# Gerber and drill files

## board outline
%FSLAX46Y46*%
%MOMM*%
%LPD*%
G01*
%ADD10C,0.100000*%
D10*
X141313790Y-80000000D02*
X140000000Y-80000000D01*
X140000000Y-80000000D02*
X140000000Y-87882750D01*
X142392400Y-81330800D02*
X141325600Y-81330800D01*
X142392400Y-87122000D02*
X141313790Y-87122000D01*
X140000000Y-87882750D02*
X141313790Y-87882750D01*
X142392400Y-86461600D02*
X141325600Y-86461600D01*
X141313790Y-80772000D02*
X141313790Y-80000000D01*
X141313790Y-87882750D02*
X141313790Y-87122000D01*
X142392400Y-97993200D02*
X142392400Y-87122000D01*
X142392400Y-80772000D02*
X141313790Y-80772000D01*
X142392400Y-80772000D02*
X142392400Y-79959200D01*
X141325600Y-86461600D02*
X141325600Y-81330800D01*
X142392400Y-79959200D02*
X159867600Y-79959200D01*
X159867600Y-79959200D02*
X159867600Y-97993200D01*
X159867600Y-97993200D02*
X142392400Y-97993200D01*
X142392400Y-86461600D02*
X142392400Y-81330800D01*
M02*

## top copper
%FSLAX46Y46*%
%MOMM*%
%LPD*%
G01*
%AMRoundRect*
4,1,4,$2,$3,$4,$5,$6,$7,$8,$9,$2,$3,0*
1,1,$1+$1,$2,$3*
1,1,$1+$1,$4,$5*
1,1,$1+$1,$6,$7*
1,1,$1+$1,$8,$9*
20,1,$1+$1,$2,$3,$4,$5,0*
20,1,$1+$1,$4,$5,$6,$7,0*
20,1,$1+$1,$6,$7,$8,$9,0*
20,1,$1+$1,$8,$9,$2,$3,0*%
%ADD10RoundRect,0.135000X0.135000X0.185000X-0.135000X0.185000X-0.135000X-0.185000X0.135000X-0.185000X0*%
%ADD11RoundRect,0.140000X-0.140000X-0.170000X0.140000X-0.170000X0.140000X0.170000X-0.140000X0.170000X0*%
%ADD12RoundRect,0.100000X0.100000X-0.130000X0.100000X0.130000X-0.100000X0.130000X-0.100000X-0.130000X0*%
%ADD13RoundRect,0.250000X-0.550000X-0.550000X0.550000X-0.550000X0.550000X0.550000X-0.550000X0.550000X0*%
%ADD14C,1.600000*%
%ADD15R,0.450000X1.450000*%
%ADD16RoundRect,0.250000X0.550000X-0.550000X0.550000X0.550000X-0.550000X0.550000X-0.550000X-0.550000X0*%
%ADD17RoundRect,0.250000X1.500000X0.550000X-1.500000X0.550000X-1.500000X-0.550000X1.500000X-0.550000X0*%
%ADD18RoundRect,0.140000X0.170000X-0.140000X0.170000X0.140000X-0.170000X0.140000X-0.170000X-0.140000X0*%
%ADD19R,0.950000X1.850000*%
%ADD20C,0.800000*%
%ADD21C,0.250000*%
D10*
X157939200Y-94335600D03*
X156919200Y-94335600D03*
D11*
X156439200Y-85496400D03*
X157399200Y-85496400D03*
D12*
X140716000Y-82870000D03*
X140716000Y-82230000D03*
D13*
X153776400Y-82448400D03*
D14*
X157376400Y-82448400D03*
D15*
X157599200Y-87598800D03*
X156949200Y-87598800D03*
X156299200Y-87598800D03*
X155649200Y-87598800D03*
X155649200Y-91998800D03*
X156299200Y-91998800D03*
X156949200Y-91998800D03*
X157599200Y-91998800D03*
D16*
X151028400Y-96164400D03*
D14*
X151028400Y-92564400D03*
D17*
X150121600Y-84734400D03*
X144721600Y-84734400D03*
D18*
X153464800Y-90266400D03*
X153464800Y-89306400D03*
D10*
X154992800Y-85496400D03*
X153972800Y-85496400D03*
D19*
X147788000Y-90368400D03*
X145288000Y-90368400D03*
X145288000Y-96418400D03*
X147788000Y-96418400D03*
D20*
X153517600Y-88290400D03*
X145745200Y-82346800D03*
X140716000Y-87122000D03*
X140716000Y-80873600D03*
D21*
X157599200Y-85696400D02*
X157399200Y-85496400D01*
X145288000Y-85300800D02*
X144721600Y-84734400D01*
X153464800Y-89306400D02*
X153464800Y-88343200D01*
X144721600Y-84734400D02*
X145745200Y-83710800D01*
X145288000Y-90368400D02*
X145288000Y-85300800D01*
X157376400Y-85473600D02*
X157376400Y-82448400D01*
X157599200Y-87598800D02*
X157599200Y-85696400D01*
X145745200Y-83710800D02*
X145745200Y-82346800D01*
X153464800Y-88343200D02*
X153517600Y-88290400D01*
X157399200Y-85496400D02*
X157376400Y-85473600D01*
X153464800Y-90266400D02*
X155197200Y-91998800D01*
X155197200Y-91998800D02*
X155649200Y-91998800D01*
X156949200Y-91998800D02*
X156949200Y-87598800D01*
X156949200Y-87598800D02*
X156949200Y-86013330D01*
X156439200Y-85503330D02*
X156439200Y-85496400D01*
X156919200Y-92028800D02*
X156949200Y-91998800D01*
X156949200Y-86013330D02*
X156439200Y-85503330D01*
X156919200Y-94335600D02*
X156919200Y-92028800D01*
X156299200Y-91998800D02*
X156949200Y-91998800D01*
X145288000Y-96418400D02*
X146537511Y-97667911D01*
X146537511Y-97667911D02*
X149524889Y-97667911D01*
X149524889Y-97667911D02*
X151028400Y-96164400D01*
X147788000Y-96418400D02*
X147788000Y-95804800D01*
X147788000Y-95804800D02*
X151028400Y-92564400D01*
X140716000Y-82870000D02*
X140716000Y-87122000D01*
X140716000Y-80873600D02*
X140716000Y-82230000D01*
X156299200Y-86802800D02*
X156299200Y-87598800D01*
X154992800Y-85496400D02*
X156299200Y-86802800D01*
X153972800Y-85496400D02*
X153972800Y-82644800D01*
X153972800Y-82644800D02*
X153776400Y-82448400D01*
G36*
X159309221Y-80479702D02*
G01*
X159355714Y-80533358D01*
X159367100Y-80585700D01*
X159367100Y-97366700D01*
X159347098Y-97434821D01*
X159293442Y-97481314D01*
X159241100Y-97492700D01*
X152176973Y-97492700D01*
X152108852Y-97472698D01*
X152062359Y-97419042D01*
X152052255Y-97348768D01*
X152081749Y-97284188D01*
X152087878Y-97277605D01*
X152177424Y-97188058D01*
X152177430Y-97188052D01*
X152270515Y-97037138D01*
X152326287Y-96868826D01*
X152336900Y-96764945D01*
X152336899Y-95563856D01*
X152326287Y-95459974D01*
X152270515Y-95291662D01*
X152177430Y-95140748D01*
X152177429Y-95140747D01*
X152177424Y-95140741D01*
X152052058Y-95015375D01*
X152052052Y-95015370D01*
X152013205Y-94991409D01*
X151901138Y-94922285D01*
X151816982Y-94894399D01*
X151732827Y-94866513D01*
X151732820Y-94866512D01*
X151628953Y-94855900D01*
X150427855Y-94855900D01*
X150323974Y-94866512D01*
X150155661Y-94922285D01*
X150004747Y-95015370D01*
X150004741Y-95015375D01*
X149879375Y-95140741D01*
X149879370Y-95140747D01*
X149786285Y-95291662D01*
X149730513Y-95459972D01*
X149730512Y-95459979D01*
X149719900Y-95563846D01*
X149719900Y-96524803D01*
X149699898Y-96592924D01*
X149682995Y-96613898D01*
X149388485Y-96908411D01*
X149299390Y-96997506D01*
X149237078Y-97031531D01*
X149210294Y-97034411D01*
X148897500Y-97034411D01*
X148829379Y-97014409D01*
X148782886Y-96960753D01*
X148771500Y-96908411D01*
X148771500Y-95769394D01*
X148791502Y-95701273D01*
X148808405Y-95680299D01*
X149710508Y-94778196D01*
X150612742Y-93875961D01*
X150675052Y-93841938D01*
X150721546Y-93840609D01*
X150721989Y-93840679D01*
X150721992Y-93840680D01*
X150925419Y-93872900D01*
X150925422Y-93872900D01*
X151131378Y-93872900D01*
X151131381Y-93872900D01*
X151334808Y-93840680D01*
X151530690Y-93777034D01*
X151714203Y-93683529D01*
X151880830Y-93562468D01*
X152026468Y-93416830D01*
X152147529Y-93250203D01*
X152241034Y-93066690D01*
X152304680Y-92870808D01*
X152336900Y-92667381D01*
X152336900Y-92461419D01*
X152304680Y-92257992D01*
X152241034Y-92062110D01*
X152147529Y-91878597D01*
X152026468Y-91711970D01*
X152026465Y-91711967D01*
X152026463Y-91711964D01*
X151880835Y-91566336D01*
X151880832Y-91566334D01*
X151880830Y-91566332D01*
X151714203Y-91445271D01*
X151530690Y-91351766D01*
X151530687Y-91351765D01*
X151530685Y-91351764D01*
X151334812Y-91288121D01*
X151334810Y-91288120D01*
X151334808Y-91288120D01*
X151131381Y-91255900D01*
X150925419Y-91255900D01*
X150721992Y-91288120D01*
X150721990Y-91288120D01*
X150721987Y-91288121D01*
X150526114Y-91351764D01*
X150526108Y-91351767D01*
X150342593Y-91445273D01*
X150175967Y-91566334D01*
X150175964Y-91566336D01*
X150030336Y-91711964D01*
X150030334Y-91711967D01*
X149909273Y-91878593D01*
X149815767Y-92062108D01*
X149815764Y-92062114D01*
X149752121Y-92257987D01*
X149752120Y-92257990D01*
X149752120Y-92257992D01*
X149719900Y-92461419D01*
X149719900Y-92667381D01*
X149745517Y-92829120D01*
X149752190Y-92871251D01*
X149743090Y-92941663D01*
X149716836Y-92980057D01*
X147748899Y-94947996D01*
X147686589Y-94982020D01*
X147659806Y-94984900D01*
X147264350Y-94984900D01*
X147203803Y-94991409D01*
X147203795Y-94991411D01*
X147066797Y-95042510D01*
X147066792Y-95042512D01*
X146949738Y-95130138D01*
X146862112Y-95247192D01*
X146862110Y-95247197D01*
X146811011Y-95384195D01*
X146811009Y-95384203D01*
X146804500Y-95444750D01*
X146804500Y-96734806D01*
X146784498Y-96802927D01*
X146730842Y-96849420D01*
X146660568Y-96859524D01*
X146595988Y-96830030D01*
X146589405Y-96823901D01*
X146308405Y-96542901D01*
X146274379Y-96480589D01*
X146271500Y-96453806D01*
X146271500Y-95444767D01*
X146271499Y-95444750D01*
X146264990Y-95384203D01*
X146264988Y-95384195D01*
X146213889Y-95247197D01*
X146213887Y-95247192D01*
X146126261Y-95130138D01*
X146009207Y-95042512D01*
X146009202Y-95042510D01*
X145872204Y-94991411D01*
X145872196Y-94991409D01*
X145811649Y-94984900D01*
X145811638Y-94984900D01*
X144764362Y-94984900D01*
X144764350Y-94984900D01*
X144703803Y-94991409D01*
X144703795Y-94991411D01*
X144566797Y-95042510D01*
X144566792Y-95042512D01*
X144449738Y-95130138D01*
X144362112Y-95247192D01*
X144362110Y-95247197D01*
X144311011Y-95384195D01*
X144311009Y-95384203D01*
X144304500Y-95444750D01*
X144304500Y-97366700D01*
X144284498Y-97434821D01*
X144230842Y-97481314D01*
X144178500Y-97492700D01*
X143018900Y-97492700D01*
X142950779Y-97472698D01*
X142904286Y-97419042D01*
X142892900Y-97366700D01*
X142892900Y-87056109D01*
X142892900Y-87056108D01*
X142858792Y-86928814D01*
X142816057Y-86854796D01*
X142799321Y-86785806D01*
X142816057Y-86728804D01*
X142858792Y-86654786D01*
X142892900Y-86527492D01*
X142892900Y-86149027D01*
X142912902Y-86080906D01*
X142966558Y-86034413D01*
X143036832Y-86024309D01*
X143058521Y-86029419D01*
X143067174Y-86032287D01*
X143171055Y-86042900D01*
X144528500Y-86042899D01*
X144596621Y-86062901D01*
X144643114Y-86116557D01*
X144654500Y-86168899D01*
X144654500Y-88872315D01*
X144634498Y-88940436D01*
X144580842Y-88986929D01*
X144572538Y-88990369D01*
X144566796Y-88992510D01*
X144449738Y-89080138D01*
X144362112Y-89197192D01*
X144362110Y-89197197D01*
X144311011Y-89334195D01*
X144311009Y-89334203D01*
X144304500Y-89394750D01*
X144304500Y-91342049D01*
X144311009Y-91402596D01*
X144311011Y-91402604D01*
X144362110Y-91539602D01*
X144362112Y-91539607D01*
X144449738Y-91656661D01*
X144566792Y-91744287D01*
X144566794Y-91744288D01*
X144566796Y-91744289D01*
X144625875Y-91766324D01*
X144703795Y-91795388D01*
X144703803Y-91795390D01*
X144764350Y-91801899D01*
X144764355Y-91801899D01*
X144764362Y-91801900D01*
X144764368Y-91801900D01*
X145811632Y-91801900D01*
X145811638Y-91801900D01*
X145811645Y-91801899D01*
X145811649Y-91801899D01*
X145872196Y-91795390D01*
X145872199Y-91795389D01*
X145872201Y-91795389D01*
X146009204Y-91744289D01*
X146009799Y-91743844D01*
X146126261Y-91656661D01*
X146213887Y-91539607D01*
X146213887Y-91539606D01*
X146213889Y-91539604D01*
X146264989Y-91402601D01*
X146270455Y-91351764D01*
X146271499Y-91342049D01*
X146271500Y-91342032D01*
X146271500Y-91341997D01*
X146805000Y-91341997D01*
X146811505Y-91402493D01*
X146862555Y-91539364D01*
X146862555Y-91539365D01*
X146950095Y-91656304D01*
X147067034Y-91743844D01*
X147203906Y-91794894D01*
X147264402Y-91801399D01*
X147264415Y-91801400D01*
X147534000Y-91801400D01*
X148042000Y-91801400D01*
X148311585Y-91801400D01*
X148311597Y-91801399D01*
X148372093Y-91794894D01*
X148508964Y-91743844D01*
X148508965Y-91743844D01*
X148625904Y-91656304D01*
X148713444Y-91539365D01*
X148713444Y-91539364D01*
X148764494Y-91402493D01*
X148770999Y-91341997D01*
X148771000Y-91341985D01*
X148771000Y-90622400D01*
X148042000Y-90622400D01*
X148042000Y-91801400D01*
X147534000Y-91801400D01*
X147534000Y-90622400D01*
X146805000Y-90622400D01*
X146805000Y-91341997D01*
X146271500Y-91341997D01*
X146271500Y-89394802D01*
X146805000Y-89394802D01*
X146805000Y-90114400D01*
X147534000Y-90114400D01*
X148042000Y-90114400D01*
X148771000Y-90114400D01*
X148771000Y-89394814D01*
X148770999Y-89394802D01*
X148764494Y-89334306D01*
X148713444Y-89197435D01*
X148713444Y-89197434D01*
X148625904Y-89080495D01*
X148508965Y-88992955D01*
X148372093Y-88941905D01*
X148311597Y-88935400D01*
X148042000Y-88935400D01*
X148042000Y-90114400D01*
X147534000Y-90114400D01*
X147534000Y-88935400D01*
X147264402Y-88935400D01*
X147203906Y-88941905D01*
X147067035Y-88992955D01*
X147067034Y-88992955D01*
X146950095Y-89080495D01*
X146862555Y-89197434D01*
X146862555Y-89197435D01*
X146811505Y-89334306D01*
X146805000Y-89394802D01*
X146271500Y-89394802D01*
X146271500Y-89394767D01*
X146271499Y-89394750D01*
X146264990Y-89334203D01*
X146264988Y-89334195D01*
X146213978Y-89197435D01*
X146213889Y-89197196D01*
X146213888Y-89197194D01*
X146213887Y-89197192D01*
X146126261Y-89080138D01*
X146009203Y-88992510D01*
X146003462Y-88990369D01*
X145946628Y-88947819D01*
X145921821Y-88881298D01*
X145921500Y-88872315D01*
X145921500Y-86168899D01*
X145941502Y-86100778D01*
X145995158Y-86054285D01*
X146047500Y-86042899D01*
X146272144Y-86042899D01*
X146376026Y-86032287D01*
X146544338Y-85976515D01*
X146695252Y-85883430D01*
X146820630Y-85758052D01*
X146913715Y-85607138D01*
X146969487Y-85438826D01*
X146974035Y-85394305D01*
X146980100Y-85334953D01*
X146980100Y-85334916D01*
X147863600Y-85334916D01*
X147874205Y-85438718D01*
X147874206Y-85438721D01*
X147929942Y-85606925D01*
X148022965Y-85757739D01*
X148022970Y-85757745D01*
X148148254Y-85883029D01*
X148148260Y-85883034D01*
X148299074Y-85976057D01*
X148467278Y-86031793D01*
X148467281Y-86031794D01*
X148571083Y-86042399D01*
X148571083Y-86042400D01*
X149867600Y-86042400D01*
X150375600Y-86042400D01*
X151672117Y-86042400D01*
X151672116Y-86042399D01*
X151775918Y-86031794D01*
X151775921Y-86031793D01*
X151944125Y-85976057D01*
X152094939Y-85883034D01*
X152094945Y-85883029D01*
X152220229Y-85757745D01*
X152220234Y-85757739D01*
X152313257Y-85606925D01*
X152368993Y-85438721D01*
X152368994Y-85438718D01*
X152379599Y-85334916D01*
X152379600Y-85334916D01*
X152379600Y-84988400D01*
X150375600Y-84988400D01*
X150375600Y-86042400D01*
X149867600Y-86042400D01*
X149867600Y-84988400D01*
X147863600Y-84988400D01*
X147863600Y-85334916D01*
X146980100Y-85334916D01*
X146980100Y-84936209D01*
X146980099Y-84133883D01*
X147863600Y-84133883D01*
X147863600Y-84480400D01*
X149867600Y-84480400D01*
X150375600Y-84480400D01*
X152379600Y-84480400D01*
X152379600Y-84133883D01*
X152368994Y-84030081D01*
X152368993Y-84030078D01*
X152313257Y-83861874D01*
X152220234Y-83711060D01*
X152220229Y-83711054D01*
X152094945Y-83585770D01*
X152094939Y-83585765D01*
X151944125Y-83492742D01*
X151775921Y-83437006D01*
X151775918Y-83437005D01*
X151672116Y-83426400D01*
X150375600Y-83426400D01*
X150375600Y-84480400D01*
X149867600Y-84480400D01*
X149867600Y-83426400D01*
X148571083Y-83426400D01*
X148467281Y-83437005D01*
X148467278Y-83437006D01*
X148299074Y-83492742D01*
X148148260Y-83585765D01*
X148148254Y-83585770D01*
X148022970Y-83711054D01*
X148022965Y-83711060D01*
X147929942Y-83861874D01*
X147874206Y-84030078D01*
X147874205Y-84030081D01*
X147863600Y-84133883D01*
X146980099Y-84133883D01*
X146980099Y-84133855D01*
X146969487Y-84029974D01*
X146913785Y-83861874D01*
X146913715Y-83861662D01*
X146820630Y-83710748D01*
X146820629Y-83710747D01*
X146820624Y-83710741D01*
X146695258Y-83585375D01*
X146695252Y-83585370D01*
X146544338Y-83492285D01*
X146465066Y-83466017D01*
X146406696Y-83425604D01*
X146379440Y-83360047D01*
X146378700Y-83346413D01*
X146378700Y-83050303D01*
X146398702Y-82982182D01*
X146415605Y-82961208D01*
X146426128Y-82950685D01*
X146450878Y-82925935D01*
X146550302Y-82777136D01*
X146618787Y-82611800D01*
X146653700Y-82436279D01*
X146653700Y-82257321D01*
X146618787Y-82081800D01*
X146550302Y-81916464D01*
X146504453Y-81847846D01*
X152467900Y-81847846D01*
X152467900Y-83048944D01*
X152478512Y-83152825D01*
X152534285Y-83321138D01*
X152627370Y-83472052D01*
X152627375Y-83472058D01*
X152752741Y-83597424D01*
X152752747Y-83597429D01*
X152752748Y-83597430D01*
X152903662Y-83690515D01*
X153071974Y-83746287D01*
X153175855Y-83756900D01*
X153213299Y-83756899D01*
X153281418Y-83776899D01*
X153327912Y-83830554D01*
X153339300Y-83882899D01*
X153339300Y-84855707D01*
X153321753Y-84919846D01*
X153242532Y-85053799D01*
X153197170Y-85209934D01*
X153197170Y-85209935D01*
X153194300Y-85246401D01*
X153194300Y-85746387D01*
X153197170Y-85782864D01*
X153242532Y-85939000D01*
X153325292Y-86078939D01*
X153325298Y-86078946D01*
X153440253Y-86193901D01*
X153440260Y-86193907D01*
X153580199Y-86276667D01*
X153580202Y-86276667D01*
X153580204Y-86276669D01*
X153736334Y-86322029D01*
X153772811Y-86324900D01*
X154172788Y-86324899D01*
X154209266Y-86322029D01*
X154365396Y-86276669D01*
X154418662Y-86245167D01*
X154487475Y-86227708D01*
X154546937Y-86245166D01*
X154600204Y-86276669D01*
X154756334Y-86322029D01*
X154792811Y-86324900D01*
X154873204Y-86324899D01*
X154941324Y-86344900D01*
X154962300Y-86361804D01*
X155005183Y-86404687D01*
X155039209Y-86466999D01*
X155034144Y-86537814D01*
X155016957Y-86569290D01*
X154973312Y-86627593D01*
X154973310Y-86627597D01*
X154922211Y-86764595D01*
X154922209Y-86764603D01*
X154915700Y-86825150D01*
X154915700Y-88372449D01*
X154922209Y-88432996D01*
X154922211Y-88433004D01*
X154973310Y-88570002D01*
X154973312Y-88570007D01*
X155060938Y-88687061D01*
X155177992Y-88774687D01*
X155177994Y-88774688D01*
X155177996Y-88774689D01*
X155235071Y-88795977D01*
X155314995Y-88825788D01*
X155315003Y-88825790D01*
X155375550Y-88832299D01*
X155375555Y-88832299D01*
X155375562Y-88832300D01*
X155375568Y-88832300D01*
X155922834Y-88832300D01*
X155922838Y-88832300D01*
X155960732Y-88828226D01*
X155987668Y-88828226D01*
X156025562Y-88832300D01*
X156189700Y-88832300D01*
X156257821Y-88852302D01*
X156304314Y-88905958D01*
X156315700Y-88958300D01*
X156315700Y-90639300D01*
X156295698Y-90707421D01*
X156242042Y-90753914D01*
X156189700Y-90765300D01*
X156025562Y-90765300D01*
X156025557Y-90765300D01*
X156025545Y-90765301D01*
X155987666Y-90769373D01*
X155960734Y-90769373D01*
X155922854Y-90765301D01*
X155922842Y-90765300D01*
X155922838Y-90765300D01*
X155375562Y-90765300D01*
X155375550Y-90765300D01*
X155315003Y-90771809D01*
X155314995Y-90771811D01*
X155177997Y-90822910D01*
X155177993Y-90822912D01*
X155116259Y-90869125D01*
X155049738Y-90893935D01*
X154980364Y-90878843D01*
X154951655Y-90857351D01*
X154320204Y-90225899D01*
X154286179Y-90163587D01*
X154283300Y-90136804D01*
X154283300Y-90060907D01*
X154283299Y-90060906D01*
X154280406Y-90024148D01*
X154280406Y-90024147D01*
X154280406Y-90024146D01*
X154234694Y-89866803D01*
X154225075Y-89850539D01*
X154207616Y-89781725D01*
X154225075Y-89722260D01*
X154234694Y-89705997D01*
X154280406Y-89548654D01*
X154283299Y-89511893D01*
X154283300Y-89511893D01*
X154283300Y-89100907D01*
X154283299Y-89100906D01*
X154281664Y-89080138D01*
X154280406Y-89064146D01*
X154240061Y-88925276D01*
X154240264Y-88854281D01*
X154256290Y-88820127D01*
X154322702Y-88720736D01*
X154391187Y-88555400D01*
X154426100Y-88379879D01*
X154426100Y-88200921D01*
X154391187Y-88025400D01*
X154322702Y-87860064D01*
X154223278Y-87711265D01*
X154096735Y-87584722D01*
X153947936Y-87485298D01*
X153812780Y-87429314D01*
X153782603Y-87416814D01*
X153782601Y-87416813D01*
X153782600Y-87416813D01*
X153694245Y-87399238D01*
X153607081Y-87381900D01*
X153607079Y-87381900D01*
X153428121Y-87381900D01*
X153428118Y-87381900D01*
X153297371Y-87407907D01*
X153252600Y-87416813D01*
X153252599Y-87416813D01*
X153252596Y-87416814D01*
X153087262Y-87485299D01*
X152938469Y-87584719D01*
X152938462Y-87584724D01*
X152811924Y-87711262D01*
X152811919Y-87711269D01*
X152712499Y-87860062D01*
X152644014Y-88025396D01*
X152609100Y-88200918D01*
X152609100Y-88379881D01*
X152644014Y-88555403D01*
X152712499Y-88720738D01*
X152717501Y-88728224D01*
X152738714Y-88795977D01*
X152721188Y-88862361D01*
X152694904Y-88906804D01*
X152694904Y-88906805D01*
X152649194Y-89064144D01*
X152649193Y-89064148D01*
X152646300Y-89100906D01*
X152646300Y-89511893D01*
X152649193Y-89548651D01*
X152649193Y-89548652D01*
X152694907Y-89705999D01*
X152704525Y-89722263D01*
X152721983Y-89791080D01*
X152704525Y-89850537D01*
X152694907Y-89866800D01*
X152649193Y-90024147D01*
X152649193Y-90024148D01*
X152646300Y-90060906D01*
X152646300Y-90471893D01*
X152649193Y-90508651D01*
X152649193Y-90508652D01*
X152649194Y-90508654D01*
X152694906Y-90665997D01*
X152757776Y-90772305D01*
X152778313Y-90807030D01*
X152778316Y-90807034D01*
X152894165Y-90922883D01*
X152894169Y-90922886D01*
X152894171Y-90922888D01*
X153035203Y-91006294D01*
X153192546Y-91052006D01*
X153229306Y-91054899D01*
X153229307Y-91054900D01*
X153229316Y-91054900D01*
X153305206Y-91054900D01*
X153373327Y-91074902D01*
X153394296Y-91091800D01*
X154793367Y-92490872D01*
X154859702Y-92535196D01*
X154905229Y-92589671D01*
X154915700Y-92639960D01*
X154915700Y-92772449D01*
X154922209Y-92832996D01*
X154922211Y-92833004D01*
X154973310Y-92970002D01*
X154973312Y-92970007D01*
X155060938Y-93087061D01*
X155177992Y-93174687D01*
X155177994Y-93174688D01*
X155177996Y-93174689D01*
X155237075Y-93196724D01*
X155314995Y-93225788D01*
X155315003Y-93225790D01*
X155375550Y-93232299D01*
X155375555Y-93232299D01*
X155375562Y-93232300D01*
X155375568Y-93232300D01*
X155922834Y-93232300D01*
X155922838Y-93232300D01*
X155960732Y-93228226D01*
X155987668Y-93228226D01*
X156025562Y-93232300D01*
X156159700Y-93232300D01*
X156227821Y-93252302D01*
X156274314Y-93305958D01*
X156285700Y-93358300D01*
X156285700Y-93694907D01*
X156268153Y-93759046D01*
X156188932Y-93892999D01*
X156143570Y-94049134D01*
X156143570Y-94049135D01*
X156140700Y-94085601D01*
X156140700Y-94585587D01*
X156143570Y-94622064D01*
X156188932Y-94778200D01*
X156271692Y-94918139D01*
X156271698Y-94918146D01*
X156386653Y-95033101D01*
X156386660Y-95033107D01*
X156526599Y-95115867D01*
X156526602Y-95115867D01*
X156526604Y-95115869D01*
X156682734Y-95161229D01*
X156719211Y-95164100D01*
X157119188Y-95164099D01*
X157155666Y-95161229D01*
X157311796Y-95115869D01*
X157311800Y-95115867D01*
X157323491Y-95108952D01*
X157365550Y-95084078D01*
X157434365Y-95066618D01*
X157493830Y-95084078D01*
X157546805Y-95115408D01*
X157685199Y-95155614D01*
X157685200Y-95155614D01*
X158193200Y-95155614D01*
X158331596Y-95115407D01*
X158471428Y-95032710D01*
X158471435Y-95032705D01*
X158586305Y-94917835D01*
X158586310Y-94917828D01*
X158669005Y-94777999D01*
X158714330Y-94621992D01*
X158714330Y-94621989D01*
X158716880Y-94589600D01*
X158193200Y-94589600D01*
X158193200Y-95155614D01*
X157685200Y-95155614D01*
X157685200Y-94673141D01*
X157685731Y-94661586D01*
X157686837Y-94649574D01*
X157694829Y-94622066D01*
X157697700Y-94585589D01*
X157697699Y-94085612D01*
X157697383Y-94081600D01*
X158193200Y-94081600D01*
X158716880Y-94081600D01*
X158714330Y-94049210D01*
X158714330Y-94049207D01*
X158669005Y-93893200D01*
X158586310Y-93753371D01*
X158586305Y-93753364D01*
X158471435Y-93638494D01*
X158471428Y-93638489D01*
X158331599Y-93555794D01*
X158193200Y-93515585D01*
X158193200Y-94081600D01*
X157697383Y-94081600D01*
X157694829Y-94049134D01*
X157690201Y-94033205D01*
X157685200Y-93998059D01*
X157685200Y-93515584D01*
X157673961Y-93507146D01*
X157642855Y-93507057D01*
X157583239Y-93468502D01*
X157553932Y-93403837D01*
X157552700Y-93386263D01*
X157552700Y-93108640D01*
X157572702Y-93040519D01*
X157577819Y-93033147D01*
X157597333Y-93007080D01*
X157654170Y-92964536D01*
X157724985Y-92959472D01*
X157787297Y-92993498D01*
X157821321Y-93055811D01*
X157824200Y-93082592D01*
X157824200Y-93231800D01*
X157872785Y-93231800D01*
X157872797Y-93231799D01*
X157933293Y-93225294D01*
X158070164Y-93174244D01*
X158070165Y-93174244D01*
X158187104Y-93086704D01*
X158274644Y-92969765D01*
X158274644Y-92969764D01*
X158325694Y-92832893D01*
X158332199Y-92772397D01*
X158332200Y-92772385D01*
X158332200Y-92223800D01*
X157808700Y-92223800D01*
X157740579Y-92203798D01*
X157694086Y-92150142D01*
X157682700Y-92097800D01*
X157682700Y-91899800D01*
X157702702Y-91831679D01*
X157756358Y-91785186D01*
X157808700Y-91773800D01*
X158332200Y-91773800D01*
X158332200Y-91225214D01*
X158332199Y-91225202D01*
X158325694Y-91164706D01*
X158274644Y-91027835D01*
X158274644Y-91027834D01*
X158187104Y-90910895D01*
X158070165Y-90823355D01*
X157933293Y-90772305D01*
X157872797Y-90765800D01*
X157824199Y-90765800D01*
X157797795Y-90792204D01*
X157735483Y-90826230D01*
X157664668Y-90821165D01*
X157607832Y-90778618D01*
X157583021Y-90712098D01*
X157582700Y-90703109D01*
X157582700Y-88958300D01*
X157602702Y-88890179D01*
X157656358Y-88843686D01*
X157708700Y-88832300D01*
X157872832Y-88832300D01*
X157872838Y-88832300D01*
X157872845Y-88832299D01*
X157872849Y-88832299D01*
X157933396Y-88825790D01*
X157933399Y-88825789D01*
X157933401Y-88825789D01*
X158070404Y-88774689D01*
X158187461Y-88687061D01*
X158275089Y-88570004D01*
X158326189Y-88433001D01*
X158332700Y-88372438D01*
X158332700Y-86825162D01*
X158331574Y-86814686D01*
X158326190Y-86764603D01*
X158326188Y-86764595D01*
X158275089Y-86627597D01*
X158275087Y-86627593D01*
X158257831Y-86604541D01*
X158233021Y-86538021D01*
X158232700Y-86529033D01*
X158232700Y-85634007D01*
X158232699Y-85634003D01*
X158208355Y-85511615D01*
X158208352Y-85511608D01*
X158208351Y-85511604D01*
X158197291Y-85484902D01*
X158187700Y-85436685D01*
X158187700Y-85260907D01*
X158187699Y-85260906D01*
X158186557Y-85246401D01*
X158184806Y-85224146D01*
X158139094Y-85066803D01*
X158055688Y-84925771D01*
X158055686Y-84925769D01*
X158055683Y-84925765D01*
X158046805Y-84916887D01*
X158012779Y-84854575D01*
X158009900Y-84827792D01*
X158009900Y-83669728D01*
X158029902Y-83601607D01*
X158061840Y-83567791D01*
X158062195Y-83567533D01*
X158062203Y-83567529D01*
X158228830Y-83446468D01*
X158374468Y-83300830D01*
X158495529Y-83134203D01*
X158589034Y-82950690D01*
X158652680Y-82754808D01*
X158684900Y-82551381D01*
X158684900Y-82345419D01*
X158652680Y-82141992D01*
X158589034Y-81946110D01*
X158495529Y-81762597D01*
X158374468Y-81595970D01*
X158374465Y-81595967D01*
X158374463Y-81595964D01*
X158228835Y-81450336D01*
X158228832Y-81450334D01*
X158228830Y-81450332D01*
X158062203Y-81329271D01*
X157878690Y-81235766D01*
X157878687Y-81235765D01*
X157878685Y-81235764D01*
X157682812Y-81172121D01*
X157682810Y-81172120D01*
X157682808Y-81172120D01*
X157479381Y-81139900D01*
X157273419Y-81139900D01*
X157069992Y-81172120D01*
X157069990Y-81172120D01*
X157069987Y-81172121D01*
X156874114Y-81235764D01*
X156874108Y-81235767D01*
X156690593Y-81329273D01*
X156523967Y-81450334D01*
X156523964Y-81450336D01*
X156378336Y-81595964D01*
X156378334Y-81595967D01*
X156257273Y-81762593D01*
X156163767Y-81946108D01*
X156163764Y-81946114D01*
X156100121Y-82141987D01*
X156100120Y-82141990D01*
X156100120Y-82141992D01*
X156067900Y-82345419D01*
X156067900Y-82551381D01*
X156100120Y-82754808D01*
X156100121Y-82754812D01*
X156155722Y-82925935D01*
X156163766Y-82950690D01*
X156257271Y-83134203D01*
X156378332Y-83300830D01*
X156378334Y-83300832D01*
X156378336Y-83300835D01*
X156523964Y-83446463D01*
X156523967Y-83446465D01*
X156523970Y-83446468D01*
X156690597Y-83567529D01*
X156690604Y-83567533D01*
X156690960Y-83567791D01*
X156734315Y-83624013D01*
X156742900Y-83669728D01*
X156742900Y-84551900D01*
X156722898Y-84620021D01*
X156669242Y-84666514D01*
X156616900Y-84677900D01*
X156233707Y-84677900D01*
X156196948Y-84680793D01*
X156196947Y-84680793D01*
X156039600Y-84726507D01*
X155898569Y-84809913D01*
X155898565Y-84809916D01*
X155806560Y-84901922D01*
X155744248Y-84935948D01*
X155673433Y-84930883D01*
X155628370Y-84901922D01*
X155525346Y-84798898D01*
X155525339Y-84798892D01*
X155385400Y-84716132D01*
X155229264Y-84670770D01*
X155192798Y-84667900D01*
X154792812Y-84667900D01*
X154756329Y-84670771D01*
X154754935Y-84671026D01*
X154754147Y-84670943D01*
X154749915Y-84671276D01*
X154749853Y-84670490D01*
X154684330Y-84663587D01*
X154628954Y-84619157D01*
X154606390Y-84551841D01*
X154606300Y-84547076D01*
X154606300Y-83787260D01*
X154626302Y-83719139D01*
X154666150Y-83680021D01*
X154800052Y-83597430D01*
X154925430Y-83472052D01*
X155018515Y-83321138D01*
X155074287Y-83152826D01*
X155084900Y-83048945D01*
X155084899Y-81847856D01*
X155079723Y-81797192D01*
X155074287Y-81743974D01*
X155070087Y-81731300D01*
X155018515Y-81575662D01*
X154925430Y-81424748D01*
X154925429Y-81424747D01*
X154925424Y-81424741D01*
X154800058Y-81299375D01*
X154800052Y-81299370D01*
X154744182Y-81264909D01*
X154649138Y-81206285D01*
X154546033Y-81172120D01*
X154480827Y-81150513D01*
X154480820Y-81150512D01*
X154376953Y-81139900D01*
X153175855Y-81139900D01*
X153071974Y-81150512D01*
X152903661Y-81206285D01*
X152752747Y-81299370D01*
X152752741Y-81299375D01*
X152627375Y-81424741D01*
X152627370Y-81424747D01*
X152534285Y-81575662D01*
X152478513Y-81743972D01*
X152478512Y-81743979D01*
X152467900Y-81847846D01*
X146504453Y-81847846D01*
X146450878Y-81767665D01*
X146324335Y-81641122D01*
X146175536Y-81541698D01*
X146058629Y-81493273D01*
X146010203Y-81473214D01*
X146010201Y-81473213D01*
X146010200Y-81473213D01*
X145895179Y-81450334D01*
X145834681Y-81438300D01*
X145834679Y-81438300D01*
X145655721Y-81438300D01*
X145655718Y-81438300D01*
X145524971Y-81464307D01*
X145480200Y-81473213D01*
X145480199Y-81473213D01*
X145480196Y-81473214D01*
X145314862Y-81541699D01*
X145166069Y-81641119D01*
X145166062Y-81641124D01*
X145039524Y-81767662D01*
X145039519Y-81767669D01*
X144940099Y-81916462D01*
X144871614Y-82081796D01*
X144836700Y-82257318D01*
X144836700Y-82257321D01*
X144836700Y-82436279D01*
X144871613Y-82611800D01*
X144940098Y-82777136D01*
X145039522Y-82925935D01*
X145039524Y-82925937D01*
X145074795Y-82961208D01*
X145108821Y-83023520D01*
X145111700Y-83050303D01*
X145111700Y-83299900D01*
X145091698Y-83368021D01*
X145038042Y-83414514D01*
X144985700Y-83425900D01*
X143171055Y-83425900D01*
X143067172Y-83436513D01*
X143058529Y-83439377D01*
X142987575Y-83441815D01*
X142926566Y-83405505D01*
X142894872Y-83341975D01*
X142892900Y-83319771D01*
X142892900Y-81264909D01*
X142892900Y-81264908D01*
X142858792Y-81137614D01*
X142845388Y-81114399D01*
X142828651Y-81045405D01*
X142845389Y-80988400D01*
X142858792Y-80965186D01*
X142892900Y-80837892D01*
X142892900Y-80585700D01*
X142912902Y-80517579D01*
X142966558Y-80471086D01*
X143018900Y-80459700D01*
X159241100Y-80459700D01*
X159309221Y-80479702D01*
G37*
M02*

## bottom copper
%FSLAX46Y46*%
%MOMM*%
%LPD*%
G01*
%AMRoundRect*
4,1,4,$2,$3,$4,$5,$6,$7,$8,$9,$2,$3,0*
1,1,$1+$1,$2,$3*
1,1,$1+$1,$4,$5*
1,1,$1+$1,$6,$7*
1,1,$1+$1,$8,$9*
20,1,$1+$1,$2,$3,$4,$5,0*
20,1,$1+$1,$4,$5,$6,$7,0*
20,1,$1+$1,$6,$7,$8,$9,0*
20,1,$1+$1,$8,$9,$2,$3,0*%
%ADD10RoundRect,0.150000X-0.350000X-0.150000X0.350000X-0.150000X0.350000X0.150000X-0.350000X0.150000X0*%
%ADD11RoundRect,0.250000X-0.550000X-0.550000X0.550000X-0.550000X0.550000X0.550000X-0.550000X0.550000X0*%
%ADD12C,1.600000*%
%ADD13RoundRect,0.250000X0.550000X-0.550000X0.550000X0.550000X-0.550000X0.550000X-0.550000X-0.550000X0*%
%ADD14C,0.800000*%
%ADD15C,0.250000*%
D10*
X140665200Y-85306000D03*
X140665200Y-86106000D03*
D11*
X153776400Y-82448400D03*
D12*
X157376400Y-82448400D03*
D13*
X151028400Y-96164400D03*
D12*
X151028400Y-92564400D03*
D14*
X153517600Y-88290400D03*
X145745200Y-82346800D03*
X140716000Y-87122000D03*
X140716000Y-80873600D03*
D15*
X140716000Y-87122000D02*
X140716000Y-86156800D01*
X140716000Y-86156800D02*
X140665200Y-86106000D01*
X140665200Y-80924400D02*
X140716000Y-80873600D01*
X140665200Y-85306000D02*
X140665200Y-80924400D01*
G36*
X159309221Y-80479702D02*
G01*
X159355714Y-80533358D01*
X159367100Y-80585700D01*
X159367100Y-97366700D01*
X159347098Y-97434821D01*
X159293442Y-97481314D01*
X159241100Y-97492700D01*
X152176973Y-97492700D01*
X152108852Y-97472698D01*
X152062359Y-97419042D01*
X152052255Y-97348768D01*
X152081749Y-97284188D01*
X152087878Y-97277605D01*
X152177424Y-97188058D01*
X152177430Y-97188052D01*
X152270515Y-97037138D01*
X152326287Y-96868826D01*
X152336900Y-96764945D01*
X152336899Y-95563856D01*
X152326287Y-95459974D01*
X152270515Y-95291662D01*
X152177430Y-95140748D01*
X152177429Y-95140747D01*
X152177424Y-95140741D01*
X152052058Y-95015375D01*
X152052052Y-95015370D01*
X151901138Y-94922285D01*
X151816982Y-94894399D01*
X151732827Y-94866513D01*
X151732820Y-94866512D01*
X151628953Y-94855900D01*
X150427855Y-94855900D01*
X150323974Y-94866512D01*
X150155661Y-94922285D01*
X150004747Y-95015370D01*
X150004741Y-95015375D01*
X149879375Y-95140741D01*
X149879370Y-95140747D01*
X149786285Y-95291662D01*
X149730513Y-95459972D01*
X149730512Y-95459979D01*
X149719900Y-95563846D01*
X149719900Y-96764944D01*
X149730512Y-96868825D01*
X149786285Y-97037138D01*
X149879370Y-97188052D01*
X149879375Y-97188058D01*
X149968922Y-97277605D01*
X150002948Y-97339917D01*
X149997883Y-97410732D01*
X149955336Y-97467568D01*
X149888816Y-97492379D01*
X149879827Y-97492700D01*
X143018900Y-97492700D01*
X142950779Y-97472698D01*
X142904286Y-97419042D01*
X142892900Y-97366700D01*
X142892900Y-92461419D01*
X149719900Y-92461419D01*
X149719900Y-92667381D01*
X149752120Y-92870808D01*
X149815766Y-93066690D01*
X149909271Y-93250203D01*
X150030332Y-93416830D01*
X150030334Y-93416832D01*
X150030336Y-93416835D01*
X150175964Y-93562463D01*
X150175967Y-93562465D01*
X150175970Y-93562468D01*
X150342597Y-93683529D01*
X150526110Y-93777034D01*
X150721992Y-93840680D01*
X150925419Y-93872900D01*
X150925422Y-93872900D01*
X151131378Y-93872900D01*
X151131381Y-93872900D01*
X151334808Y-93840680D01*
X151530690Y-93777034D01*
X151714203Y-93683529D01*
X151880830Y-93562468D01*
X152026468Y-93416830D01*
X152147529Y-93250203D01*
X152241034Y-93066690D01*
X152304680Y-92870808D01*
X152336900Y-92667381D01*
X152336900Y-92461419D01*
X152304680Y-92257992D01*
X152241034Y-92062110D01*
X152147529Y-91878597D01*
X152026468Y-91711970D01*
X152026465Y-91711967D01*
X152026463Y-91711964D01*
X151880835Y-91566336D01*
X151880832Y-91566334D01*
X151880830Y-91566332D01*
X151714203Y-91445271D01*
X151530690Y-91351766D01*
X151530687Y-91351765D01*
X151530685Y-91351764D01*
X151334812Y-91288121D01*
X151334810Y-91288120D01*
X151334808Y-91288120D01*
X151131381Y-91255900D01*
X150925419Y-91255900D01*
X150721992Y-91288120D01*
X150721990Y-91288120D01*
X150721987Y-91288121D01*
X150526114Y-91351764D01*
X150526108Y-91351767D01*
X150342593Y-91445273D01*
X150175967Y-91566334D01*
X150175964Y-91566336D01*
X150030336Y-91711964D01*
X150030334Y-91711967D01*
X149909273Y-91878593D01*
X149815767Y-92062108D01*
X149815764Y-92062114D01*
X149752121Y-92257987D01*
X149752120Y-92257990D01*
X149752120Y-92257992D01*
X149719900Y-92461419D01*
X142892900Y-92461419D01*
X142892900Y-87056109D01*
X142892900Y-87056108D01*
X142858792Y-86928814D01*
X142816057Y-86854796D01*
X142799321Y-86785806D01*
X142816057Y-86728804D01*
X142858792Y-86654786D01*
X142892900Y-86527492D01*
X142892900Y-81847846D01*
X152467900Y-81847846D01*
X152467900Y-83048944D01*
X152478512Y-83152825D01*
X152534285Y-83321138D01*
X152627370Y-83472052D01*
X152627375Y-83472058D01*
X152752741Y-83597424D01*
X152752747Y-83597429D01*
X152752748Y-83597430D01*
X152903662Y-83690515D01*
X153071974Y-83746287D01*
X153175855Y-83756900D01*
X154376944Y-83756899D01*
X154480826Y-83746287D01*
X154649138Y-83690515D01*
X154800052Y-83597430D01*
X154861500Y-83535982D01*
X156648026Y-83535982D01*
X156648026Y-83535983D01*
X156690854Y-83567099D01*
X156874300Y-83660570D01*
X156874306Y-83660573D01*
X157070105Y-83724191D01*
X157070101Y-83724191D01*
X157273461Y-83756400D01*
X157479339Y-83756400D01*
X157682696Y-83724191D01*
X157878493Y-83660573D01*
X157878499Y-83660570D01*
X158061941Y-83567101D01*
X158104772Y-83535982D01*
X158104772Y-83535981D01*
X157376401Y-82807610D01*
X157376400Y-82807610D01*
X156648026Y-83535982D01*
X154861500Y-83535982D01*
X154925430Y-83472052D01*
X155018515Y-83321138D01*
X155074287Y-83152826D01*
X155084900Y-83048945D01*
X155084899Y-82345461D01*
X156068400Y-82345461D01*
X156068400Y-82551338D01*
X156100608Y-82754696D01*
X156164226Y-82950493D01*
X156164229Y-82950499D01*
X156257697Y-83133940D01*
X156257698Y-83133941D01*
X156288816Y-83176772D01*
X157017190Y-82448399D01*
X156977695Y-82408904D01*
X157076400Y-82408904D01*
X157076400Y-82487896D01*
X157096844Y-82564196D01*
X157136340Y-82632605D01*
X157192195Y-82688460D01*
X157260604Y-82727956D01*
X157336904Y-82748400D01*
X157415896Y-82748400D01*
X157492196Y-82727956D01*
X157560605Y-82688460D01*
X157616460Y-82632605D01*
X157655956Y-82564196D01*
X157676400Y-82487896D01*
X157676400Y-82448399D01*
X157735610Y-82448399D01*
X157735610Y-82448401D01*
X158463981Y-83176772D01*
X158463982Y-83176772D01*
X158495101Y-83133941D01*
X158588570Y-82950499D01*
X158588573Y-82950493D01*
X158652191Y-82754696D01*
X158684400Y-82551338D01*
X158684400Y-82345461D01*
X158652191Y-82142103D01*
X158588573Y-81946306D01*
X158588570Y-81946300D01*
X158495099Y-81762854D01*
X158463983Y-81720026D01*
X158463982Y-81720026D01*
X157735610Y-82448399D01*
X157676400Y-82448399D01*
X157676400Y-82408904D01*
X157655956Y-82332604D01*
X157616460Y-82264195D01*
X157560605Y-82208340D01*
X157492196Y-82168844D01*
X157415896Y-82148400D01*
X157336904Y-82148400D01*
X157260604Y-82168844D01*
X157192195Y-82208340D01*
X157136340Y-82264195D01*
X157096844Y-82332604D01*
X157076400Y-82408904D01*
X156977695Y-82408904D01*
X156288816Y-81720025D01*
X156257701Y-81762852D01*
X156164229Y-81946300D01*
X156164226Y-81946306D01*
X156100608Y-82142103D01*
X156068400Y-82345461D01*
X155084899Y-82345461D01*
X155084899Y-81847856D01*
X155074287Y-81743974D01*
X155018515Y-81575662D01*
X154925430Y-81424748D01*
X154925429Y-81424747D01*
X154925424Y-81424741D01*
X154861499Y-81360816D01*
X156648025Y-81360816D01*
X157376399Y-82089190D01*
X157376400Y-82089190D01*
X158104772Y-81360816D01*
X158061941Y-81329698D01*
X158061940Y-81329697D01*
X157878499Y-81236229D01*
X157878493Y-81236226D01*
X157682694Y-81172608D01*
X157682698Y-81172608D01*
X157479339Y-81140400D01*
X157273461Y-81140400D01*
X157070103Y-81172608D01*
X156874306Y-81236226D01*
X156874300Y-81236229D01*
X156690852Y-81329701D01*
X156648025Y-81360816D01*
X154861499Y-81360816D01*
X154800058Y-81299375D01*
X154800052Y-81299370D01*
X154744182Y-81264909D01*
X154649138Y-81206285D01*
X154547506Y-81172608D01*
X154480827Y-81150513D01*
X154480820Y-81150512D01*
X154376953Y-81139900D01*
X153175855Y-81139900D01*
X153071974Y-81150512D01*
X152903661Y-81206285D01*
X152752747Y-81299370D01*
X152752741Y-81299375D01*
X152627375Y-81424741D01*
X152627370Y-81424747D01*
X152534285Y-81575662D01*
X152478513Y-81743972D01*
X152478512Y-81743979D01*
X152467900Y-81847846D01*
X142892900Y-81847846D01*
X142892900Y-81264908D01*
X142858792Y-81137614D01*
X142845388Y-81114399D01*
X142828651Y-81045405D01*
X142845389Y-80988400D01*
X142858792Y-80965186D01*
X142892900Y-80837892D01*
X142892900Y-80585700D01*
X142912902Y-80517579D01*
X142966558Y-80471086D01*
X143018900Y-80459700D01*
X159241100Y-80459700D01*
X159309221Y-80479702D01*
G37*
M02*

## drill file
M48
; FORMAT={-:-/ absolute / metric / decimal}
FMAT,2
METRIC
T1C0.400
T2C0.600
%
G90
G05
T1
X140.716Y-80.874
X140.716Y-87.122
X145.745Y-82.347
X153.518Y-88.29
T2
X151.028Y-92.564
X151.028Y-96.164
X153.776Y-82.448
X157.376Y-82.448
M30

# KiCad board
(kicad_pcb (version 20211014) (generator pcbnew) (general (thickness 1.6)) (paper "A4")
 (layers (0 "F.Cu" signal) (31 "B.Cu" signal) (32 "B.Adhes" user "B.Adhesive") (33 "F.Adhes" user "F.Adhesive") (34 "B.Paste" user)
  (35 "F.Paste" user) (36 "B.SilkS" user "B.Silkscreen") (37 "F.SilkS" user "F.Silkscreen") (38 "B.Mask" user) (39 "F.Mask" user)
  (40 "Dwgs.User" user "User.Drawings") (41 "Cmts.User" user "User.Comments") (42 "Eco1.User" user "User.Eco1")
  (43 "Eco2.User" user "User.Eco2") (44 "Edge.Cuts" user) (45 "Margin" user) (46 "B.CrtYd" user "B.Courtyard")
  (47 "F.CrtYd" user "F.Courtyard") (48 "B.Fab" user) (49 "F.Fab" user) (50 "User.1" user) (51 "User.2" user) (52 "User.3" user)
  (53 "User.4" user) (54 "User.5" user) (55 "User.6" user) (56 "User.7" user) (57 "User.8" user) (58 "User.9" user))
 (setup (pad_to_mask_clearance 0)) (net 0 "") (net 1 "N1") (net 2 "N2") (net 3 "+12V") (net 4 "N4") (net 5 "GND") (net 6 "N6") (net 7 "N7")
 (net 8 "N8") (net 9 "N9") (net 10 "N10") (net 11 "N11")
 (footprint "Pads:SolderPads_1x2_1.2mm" (layer "F.Cu") (at 140.6652 85.706)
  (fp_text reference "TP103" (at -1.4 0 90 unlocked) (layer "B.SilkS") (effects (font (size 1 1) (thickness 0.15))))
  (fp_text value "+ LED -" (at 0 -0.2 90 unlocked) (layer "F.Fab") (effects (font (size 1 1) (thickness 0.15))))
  (pad "1" smd roundrect (at 0 -0.4) (size 1 0.6) (layers "B.Cu" "B.Paste" "B.Mask") (roundrect_rratio 0.25) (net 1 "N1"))
  (pad "2" smd roundrect (at 0 0.4) (size 1 0.6) (layers "B.Cu" "B.Paste" "B.Mask") (roundrect_rratio 0.25) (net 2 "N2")))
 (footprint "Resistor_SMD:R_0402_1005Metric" (layer "F.Cu") (at 157.4292 94.3356 180)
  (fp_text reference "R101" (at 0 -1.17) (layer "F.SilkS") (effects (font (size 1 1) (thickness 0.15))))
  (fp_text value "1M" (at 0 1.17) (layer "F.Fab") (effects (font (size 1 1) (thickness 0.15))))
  (pad "1" smd roundrect (at -0.51 0 180) (size 0.54 0.64) (layers "F.Cu" "F.Paste" "F.Mask") (roundrect_rratio 0.25) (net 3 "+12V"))
  (pad "2" smd roundrect (at 0.51 0 180) (size 0.54 0.64) (layers "F.Cu" "F.Paste" "F.Mask") (roundrect_rratio 0.25) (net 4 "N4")))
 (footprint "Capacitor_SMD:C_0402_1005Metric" (layer "F.Cu") (at 156.9192 85.4964)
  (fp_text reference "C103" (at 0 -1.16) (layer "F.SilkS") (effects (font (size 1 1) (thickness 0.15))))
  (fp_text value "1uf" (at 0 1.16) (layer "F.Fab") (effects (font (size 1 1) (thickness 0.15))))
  (pad "1" smd roundrect (at -0.48 0) (size 0.56 0.62) (layers "F.Cu" "F.Paste" "F.Mask") (roundrect_rratio 0.25) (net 4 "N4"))
  (pad "2" smd roundrect (at 0.48 0) (size 0.56 0.62) (layers "F.Cu" "F.Paste" "F.Mask") (roundrect_rratio 0.25) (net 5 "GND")))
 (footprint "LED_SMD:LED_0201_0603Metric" (layer "F.Cu") (at 140.716 82.55 90)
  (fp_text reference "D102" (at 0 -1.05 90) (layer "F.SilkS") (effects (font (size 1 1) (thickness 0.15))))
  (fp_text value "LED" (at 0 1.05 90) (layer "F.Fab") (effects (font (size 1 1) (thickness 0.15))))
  (pad "" smd roundrect (at 0.345 0 90) (size 0.318 0.36) (layers "F.Paste") (roundrect_rratio 0.25))
  (pad "" smd roundrect (at -0.345 0 90) (size 0.318 0.36) (layers "F.Paste") (roundrect_rratio 0.25))
  (pad "1" smd roundrect (at -0.32 0 90) (size 0.46 0.4) (layers "F.Cu" "F.Mask") (roundrect_rratio 0.25) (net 2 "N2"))
  (pad "2" smd roundrect (at 0.32 0 90) (size 0.46 0.4) (layers "F.Cu" "F.Mask") (roundrect_rratio 0.25) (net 1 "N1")))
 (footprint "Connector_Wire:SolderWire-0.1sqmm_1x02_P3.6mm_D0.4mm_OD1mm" (layer "F.Cu") (at 153.7764 82.4484)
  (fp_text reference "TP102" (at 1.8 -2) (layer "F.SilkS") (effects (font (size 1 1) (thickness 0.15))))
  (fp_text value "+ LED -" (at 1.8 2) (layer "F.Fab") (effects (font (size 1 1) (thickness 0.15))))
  (pad "1" thru_hole roundrect (at 0 0) (size 1.6 1.6) (drill 0.6) (layers *.Cu *.Mask) (roundrect_rratio 0.15625) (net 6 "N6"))
  (pad "2" thru_hole circle (at 3.6 0) (size 1.6 1.6) (drill 0.6) (layers *.Cu *.Mask) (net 5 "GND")))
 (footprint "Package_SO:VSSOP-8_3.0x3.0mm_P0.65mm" (layer "F.Cu") (at 156.6242 89.7988 -90)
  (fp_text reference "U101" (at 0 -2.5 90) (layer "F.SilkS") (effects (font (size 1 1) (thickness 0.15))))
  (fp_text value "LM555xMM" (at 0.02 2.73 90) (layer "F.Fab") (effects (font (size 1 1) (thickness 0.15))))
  (pad "1" smd rect (at -2.2 -0.975 180) (size 0.45 1.45) (layers "F.Cu" "F.Paste" "F.Mask") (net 5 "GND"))
  (pad "2" smd rect (at -2.2 -0.325 180) (size 0.45 1.45) (layers "F.Cu" "F.Paste" "F.Mask") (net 4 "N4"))
  (pad "3" smd rect (at -2.2 0.325 180) (size 0.45 1.45) (layers "F.Cu" "F.Paste" "F.Mask") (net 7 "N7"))
  (pad "4" smd rect (at -2.2 0.975 180) (size 0.45 1.45) (layers "F.Cu" "F.Paste" "F.Mask") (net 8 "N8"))
  (pad "5" smd rect (at 2.2 0.975 180) (size 0.45 1.45) (layers "F.Cu" "F.Paste" "F.Mask") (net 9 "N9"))
  (pad "6" smd rect (at 2.2 0.325 180) (size 0.45 1.45) (layers "F.Cu" "F.Paste" "F.Mask") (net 4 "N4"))
  (pad "7" smd rect (at 2.2 -0.325 180) (size 0.45 1.45) (layers "F.Cu" "F.Paste" "F.Mask") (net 4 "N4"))
  (pad "8" smd rect (at 2.2 -0.975 180) (size 0.45 1.45) (layers "F.Cu" "F.Paste" "F.Mask") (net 3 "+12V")))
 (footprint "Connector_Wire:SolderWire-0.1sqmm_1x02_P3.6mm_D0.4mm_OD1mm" (layer "F.Cu") (at 151.0284 96.1644 90)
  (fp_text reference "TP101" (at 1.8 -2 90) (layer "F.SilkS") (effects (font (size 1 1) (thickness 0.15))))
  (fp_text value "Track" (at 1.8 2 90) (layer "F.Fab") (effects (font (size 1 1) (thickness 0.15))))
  (pad "1" thru_hole roundrect (at 0 0 90) (size 1.6 1.6) (drill 0.6) (layers *.Cu *.Mask) (roundrect_rratio 0.15625) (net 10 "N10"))
  (pad "2" thru_hole circle (at 3.6 0 90) (size 1.6 1.6) (drill 0.6) (layers *.Cu *.Mask) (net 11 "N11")))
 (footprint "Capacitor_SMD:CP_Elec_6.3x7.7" (layer "F.Cu") (at 147.4216 84.7344 180)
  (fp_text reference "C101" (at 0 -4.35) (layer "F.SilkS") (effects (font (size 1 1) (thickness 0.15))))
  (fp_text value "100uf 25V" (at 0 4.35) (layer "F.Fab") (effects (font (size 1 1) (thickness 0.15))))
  (pad "1" smd roundrect (at -2.7 0 180) (size 3.5 1.6) (layers "F.Cu" "F.Paste" "F.Mask") (roundrect_rratio 0.15625) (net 3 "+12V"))
  (pad "2" smd roundrect (at 2.7 0 180) (size 3.5 1.6) (layers "F.Cu" "F.Paste" "F.Mask") (roundrect_rratio 0.15625) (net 5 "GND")))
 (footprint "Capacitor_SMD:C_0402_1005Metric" (layer "F.Cu") (at 153.4648 89.7864 90)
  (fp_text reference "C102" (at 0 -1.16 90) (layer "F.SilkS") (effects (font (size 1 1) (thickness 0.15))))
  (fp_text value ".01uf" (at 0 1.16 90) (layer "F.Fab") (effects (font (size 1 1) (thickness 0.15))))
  (pad "1" smd roundrect (at -0.48 0 90) (size 0.56 0.62) (layers "F.Cu" "F.Paste" "F.Mask") (roundrect_rratio 0.25) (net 9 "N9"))
  (pad "2" smd roundrect (at 0.48 0 90) (size 0.56 0.62) (layers "F.Cu" "F.Paste" "F.Mask") (roundrect_rratio 0.25) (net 5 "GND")))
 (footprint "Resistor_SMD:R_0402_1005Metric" (layer "F.Cu") (at 154.4828 85.4964 180)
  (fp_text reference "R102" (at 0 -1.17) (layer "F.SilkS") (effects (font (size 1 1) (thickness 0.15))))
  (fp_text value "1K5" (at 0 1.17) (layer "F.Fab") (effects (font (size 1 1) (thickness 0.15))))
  (pad "1" smd roundrect (at -0.51 0 180) (size 0.54 0.64) (layers "F.Cu" "F.Paste" "F.Mask") (roundrect_rratio 0.25) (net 7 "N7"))
  (pad "2" smd roundrect (at 0.51 0 180) (size 0.54 0.64) (layers "F.Cu" "F.Paste" "F.Mask") (roundrect_rratio 0.25) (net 6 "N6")))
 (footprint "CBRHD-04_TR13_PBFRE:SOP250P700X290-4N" (layer "F.Cu") (at 146.538 93.3934 -90)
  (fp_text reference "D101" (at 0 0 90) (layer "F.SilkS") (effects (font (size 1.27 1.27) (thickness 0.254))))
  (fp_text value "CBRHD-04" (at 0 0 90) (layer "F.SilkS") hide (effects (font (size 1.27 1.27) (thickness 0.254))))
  (pad "1" smd rect locked (at -3.025 -1.25) (size 0.95 1.85) (layers "F.Cu" "F.Paste" "F.Mask") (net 3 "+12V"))
  (pad "2" smd rect locked (at -3.025 1.25) (size 0.95 1.85) (layers "F.Cu" "F.Paste" "F.Mask") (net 5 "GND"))
  (pad "3" smd rect locked (at 3.025 1.25) (size 0.95 1.85) (layers "F.Cu" "F.Paste" "F.Mask") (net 10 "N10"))
  (pad "4" smd rect locked (at 3.025 -1.25) (size 0.95 1.85) (layers "F.Cu" "F.Paste" "F.Mask") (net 11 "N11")))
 (gr_line (start 141.31379 80) (end 140 80) (layer "Edge.Cuts") (width 0.1))
 (gr_line (start 140 80) (end 140 87.88275) (layer "Edge.Cuts") (width 0.1))
 (gr_line (start 142.3924 81.3308) (end 141.3256 81.3308) (layer "Edge.Cuts") (width 0.1))
 (gr_line (start 142.3924 87.122) (end 141.31379 87.122) (layer "Edge.Cuts") (width 0.1))
 (gr_line (start 140 87.88275) (end 141.31379 87.88275) (layer "Edge.Cuts") (width 0.1))
 (gr_line (start 142.3924 86.4616) (end 141.3256 86.4616) (layer "Edge.Cuts") (width 0.1))
 (gr_line (start 141.31379 80.772) (end 141.31379 80) (layer "Edge.Cuts") (width 0.1))
 (gr_line (start 141.31379 87.88275) (end 141.31379 87.122) (layer "Edge.Cuts") (width 0.1))
 (gr_line (start 142.3924 97.9932) (end 142.3924 87.122) (layer "Edge.Cuts") (width 0.1))
 (gr_line (start 142.3924 80.772) (end 141.31379 80.772) (layer "Edge.Cuts") (width 0.1))
 (gr_line (start 142.3924 80.772) (end 142.3924 79.9592) (layer "Edge.Cuts") (width 0.1))
 (gr_line (start 141.3256 86.4616) (end 141.3256 81.3308) (layer "Edge.Cuts") (width 0.1))
 (gr_line (start 142.3924 79.9592) (end 159.8676 79.9592) (layer "Edge.Cuts") (width 0.1))
 (gr_line (start 159.8676 79.9592) (end 159.8676 97.9932) (layer "Edge.Cuts") (width 0.1))
 (gr_line (start 159.8676 97.9932) (end 142.3924 97.9932) (layer "Edge.Cuts") (width 0.1))
 (gr_line (start 142.3924 86.4616) (end 142.3924 81.3308) (layer "Edge.Cuts") (width 0.1))
 (segment (start 157.5992 85.6964) (end 157.3992 85.4964) (width 0.25) (layer "F.Cu") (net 5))
 (segment (start 145.288 85.3008) (end 144.7216 84.7344) (width 0.25) (layer "F.Cu") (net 5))
 (segment (start 153.4648 89.3064) (end 153.4648 88.3432) (width 0.25) (layer "F.Cu") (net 5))
 (segment (start 144.7216 84.7344) (end 145.7452 83.7108) (width 0.25) (layer "F.Cu") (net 5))
 (segment (start 145.288 90.3684) (end 145.288 85.3008) (width 0.25) (layer "F.Cu") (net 5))
 (segment (start 157.3764 85.4736) (end 157.3764 82.4484) (width 0.25) (layer "F.Cu") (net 5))
 (segment (start 157.5992 87.5988) (end 157.5992 85.6964) (width 0.25) (layer "F.Cu") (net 5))
 (segment (start 145.7452 83.7108) (end 145.7452 82.3468) (width 0.25) (layer "F.Cu") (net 5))
 (segment (start 153.4648 88.3432) (end 153.5176 88.2904) (width 0.25) (layer "F.Cu") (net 5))
 (segment (start 157.3992 85.4964) (end 157.3764 85.4736) (width 0.25) (layer "F.Cu") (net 5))
 (via (at 153.5176 88.2904) (size 0.8) (drill 0.4) (layers "F.Cu" "B.Cu") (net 5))
 (via (at 145.7452 82.3468) (size 0.8) (drill 0.4) (layers "F.Cu" "B.Cu") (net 5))
 (segment (start 153.4648 90.2664) (end 155.1972 91.9988) (width 0.25) (layer "F.Cu") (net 9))
 (segment (start 155.1972 91.9988) (end 155.6492 91.9988) (width 0.25) (layer "F.Cu") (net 9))
 (segment (start 156.9492 91.9988) (end 156.9492 87.5988) (width 0.25) (layer "F.Cu") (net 4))
 (segment (start 156.9492 87.5988) (end 156.9492 86.01333) (width 0.25) (layer "F.Cu") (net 4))
 (segment (start 156.4392 85.50333) (end 156.4392 85.4964) (width 0.25) (layer "F.Cu") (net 4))
 (segment (start 156.9192 92.0288) (end 156.9492 91.9988) (width 0.25) (layer "F.Cu") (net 4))
 (segment (start 156.9492 86.01333) (end 156.4392 85.50333) (width 0.25) (layer "F.Cu") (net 4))
 (segment (start 156.9192 94.3356) (end 156.9192 92.0288) (width 0.25) (layer "F.Cu") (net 4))
 (segment (start 156.2992 91.9988) (end 156.9492 91.9988) (width 0.25) (layer "F.Cu") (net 4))
 (segment (start 145.288 96.4184) (end 146.537511 97.667911) (width 0.25) (layer "F.Cu") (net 10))
 (segment (start 146.537511 97.667911) (end 149.524889 97.667911) (width 0.25) (layer "F.Cu") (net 10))
 (segment (start 149.524889 97.667911) (end 151.0284 96.1644) (width 0.25) (layer "F.Cu") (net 10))
 (segment (start 147.788 96.4184) (end 147.788 95.8048) (width 0.25) (layer "F.Cu") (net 11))
 (segment (start 147.788 95.8048) (end 151.0284 92.5644) (width 0.25) (layer "F.Cu") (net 11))
 (segment (start 140.716 82.87) (end 140.716 87.122) (width 0.25) (layer "F.Cu") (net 2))
 (via (at 140.716 87.122) (size 0.8) (drill 0.4) (layers "F.Cu" "B.Cu") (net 2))
 (segment (start 140.716 87.122) (end 140.716 86.1568) (width 0.25) (layer "B.Cu") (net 2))
 (segment (start 140.716 86.1568) (end 140.6652 86.106) (width 0.25) (layer "B.Cu") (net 2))
 (segment (start 140.716 80.8736) (end 140.716 82.23) (width 0.25) (layer "F.Cu") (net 1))
 (via (at 140.716 80.8736) (size 0.8) (drill 0.4) (layers "F.Cu" "B.Cu") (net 1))
 (segment (start 140.6652 80.9244) (end 140.716 80.8736) (width 0.25) (layer "B.Cu") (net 1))
 (segment (start 140.6652 85.306) (end 140.6652 80.9244) (width 0.25) (layer "B.Cu") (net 1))
 (segment (start 156.2992 86.8028) (end 156.2992 87.5988) (width 0.25) (layer "F.Cu") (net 7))
 (segment (start 154.9928 85.4964) (end 156.2992 86.8028) (width 0.25) (layer "F.Cu") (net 7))
 (segment (start 153.9728 85.4964) (end 153.9728 82.6448) (width 0.25) (layer "F.Cu") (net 6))
 (segment (start 153.9728 82.6448) (end 153.7764 82.4484) (width 0.25) (layer "F.Cu") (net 6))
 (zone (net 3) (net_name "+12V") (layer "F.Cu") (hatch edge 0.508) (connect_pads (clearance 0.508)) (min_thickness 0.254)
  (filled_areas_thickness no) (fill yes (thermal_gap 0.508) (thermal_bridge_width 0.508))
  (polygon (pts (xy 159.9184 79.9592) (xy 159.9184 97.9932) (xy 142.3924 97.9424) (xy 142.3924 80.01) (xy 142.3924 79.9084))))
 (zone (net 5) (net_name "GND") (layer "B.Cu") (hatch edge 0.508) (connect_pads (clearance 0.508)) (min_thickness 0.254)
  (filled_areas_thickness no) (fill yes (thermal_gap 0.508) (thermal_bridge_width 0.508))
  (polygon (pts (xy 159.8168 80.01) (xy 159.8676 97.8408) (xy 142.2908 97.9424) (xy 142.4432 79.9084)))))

